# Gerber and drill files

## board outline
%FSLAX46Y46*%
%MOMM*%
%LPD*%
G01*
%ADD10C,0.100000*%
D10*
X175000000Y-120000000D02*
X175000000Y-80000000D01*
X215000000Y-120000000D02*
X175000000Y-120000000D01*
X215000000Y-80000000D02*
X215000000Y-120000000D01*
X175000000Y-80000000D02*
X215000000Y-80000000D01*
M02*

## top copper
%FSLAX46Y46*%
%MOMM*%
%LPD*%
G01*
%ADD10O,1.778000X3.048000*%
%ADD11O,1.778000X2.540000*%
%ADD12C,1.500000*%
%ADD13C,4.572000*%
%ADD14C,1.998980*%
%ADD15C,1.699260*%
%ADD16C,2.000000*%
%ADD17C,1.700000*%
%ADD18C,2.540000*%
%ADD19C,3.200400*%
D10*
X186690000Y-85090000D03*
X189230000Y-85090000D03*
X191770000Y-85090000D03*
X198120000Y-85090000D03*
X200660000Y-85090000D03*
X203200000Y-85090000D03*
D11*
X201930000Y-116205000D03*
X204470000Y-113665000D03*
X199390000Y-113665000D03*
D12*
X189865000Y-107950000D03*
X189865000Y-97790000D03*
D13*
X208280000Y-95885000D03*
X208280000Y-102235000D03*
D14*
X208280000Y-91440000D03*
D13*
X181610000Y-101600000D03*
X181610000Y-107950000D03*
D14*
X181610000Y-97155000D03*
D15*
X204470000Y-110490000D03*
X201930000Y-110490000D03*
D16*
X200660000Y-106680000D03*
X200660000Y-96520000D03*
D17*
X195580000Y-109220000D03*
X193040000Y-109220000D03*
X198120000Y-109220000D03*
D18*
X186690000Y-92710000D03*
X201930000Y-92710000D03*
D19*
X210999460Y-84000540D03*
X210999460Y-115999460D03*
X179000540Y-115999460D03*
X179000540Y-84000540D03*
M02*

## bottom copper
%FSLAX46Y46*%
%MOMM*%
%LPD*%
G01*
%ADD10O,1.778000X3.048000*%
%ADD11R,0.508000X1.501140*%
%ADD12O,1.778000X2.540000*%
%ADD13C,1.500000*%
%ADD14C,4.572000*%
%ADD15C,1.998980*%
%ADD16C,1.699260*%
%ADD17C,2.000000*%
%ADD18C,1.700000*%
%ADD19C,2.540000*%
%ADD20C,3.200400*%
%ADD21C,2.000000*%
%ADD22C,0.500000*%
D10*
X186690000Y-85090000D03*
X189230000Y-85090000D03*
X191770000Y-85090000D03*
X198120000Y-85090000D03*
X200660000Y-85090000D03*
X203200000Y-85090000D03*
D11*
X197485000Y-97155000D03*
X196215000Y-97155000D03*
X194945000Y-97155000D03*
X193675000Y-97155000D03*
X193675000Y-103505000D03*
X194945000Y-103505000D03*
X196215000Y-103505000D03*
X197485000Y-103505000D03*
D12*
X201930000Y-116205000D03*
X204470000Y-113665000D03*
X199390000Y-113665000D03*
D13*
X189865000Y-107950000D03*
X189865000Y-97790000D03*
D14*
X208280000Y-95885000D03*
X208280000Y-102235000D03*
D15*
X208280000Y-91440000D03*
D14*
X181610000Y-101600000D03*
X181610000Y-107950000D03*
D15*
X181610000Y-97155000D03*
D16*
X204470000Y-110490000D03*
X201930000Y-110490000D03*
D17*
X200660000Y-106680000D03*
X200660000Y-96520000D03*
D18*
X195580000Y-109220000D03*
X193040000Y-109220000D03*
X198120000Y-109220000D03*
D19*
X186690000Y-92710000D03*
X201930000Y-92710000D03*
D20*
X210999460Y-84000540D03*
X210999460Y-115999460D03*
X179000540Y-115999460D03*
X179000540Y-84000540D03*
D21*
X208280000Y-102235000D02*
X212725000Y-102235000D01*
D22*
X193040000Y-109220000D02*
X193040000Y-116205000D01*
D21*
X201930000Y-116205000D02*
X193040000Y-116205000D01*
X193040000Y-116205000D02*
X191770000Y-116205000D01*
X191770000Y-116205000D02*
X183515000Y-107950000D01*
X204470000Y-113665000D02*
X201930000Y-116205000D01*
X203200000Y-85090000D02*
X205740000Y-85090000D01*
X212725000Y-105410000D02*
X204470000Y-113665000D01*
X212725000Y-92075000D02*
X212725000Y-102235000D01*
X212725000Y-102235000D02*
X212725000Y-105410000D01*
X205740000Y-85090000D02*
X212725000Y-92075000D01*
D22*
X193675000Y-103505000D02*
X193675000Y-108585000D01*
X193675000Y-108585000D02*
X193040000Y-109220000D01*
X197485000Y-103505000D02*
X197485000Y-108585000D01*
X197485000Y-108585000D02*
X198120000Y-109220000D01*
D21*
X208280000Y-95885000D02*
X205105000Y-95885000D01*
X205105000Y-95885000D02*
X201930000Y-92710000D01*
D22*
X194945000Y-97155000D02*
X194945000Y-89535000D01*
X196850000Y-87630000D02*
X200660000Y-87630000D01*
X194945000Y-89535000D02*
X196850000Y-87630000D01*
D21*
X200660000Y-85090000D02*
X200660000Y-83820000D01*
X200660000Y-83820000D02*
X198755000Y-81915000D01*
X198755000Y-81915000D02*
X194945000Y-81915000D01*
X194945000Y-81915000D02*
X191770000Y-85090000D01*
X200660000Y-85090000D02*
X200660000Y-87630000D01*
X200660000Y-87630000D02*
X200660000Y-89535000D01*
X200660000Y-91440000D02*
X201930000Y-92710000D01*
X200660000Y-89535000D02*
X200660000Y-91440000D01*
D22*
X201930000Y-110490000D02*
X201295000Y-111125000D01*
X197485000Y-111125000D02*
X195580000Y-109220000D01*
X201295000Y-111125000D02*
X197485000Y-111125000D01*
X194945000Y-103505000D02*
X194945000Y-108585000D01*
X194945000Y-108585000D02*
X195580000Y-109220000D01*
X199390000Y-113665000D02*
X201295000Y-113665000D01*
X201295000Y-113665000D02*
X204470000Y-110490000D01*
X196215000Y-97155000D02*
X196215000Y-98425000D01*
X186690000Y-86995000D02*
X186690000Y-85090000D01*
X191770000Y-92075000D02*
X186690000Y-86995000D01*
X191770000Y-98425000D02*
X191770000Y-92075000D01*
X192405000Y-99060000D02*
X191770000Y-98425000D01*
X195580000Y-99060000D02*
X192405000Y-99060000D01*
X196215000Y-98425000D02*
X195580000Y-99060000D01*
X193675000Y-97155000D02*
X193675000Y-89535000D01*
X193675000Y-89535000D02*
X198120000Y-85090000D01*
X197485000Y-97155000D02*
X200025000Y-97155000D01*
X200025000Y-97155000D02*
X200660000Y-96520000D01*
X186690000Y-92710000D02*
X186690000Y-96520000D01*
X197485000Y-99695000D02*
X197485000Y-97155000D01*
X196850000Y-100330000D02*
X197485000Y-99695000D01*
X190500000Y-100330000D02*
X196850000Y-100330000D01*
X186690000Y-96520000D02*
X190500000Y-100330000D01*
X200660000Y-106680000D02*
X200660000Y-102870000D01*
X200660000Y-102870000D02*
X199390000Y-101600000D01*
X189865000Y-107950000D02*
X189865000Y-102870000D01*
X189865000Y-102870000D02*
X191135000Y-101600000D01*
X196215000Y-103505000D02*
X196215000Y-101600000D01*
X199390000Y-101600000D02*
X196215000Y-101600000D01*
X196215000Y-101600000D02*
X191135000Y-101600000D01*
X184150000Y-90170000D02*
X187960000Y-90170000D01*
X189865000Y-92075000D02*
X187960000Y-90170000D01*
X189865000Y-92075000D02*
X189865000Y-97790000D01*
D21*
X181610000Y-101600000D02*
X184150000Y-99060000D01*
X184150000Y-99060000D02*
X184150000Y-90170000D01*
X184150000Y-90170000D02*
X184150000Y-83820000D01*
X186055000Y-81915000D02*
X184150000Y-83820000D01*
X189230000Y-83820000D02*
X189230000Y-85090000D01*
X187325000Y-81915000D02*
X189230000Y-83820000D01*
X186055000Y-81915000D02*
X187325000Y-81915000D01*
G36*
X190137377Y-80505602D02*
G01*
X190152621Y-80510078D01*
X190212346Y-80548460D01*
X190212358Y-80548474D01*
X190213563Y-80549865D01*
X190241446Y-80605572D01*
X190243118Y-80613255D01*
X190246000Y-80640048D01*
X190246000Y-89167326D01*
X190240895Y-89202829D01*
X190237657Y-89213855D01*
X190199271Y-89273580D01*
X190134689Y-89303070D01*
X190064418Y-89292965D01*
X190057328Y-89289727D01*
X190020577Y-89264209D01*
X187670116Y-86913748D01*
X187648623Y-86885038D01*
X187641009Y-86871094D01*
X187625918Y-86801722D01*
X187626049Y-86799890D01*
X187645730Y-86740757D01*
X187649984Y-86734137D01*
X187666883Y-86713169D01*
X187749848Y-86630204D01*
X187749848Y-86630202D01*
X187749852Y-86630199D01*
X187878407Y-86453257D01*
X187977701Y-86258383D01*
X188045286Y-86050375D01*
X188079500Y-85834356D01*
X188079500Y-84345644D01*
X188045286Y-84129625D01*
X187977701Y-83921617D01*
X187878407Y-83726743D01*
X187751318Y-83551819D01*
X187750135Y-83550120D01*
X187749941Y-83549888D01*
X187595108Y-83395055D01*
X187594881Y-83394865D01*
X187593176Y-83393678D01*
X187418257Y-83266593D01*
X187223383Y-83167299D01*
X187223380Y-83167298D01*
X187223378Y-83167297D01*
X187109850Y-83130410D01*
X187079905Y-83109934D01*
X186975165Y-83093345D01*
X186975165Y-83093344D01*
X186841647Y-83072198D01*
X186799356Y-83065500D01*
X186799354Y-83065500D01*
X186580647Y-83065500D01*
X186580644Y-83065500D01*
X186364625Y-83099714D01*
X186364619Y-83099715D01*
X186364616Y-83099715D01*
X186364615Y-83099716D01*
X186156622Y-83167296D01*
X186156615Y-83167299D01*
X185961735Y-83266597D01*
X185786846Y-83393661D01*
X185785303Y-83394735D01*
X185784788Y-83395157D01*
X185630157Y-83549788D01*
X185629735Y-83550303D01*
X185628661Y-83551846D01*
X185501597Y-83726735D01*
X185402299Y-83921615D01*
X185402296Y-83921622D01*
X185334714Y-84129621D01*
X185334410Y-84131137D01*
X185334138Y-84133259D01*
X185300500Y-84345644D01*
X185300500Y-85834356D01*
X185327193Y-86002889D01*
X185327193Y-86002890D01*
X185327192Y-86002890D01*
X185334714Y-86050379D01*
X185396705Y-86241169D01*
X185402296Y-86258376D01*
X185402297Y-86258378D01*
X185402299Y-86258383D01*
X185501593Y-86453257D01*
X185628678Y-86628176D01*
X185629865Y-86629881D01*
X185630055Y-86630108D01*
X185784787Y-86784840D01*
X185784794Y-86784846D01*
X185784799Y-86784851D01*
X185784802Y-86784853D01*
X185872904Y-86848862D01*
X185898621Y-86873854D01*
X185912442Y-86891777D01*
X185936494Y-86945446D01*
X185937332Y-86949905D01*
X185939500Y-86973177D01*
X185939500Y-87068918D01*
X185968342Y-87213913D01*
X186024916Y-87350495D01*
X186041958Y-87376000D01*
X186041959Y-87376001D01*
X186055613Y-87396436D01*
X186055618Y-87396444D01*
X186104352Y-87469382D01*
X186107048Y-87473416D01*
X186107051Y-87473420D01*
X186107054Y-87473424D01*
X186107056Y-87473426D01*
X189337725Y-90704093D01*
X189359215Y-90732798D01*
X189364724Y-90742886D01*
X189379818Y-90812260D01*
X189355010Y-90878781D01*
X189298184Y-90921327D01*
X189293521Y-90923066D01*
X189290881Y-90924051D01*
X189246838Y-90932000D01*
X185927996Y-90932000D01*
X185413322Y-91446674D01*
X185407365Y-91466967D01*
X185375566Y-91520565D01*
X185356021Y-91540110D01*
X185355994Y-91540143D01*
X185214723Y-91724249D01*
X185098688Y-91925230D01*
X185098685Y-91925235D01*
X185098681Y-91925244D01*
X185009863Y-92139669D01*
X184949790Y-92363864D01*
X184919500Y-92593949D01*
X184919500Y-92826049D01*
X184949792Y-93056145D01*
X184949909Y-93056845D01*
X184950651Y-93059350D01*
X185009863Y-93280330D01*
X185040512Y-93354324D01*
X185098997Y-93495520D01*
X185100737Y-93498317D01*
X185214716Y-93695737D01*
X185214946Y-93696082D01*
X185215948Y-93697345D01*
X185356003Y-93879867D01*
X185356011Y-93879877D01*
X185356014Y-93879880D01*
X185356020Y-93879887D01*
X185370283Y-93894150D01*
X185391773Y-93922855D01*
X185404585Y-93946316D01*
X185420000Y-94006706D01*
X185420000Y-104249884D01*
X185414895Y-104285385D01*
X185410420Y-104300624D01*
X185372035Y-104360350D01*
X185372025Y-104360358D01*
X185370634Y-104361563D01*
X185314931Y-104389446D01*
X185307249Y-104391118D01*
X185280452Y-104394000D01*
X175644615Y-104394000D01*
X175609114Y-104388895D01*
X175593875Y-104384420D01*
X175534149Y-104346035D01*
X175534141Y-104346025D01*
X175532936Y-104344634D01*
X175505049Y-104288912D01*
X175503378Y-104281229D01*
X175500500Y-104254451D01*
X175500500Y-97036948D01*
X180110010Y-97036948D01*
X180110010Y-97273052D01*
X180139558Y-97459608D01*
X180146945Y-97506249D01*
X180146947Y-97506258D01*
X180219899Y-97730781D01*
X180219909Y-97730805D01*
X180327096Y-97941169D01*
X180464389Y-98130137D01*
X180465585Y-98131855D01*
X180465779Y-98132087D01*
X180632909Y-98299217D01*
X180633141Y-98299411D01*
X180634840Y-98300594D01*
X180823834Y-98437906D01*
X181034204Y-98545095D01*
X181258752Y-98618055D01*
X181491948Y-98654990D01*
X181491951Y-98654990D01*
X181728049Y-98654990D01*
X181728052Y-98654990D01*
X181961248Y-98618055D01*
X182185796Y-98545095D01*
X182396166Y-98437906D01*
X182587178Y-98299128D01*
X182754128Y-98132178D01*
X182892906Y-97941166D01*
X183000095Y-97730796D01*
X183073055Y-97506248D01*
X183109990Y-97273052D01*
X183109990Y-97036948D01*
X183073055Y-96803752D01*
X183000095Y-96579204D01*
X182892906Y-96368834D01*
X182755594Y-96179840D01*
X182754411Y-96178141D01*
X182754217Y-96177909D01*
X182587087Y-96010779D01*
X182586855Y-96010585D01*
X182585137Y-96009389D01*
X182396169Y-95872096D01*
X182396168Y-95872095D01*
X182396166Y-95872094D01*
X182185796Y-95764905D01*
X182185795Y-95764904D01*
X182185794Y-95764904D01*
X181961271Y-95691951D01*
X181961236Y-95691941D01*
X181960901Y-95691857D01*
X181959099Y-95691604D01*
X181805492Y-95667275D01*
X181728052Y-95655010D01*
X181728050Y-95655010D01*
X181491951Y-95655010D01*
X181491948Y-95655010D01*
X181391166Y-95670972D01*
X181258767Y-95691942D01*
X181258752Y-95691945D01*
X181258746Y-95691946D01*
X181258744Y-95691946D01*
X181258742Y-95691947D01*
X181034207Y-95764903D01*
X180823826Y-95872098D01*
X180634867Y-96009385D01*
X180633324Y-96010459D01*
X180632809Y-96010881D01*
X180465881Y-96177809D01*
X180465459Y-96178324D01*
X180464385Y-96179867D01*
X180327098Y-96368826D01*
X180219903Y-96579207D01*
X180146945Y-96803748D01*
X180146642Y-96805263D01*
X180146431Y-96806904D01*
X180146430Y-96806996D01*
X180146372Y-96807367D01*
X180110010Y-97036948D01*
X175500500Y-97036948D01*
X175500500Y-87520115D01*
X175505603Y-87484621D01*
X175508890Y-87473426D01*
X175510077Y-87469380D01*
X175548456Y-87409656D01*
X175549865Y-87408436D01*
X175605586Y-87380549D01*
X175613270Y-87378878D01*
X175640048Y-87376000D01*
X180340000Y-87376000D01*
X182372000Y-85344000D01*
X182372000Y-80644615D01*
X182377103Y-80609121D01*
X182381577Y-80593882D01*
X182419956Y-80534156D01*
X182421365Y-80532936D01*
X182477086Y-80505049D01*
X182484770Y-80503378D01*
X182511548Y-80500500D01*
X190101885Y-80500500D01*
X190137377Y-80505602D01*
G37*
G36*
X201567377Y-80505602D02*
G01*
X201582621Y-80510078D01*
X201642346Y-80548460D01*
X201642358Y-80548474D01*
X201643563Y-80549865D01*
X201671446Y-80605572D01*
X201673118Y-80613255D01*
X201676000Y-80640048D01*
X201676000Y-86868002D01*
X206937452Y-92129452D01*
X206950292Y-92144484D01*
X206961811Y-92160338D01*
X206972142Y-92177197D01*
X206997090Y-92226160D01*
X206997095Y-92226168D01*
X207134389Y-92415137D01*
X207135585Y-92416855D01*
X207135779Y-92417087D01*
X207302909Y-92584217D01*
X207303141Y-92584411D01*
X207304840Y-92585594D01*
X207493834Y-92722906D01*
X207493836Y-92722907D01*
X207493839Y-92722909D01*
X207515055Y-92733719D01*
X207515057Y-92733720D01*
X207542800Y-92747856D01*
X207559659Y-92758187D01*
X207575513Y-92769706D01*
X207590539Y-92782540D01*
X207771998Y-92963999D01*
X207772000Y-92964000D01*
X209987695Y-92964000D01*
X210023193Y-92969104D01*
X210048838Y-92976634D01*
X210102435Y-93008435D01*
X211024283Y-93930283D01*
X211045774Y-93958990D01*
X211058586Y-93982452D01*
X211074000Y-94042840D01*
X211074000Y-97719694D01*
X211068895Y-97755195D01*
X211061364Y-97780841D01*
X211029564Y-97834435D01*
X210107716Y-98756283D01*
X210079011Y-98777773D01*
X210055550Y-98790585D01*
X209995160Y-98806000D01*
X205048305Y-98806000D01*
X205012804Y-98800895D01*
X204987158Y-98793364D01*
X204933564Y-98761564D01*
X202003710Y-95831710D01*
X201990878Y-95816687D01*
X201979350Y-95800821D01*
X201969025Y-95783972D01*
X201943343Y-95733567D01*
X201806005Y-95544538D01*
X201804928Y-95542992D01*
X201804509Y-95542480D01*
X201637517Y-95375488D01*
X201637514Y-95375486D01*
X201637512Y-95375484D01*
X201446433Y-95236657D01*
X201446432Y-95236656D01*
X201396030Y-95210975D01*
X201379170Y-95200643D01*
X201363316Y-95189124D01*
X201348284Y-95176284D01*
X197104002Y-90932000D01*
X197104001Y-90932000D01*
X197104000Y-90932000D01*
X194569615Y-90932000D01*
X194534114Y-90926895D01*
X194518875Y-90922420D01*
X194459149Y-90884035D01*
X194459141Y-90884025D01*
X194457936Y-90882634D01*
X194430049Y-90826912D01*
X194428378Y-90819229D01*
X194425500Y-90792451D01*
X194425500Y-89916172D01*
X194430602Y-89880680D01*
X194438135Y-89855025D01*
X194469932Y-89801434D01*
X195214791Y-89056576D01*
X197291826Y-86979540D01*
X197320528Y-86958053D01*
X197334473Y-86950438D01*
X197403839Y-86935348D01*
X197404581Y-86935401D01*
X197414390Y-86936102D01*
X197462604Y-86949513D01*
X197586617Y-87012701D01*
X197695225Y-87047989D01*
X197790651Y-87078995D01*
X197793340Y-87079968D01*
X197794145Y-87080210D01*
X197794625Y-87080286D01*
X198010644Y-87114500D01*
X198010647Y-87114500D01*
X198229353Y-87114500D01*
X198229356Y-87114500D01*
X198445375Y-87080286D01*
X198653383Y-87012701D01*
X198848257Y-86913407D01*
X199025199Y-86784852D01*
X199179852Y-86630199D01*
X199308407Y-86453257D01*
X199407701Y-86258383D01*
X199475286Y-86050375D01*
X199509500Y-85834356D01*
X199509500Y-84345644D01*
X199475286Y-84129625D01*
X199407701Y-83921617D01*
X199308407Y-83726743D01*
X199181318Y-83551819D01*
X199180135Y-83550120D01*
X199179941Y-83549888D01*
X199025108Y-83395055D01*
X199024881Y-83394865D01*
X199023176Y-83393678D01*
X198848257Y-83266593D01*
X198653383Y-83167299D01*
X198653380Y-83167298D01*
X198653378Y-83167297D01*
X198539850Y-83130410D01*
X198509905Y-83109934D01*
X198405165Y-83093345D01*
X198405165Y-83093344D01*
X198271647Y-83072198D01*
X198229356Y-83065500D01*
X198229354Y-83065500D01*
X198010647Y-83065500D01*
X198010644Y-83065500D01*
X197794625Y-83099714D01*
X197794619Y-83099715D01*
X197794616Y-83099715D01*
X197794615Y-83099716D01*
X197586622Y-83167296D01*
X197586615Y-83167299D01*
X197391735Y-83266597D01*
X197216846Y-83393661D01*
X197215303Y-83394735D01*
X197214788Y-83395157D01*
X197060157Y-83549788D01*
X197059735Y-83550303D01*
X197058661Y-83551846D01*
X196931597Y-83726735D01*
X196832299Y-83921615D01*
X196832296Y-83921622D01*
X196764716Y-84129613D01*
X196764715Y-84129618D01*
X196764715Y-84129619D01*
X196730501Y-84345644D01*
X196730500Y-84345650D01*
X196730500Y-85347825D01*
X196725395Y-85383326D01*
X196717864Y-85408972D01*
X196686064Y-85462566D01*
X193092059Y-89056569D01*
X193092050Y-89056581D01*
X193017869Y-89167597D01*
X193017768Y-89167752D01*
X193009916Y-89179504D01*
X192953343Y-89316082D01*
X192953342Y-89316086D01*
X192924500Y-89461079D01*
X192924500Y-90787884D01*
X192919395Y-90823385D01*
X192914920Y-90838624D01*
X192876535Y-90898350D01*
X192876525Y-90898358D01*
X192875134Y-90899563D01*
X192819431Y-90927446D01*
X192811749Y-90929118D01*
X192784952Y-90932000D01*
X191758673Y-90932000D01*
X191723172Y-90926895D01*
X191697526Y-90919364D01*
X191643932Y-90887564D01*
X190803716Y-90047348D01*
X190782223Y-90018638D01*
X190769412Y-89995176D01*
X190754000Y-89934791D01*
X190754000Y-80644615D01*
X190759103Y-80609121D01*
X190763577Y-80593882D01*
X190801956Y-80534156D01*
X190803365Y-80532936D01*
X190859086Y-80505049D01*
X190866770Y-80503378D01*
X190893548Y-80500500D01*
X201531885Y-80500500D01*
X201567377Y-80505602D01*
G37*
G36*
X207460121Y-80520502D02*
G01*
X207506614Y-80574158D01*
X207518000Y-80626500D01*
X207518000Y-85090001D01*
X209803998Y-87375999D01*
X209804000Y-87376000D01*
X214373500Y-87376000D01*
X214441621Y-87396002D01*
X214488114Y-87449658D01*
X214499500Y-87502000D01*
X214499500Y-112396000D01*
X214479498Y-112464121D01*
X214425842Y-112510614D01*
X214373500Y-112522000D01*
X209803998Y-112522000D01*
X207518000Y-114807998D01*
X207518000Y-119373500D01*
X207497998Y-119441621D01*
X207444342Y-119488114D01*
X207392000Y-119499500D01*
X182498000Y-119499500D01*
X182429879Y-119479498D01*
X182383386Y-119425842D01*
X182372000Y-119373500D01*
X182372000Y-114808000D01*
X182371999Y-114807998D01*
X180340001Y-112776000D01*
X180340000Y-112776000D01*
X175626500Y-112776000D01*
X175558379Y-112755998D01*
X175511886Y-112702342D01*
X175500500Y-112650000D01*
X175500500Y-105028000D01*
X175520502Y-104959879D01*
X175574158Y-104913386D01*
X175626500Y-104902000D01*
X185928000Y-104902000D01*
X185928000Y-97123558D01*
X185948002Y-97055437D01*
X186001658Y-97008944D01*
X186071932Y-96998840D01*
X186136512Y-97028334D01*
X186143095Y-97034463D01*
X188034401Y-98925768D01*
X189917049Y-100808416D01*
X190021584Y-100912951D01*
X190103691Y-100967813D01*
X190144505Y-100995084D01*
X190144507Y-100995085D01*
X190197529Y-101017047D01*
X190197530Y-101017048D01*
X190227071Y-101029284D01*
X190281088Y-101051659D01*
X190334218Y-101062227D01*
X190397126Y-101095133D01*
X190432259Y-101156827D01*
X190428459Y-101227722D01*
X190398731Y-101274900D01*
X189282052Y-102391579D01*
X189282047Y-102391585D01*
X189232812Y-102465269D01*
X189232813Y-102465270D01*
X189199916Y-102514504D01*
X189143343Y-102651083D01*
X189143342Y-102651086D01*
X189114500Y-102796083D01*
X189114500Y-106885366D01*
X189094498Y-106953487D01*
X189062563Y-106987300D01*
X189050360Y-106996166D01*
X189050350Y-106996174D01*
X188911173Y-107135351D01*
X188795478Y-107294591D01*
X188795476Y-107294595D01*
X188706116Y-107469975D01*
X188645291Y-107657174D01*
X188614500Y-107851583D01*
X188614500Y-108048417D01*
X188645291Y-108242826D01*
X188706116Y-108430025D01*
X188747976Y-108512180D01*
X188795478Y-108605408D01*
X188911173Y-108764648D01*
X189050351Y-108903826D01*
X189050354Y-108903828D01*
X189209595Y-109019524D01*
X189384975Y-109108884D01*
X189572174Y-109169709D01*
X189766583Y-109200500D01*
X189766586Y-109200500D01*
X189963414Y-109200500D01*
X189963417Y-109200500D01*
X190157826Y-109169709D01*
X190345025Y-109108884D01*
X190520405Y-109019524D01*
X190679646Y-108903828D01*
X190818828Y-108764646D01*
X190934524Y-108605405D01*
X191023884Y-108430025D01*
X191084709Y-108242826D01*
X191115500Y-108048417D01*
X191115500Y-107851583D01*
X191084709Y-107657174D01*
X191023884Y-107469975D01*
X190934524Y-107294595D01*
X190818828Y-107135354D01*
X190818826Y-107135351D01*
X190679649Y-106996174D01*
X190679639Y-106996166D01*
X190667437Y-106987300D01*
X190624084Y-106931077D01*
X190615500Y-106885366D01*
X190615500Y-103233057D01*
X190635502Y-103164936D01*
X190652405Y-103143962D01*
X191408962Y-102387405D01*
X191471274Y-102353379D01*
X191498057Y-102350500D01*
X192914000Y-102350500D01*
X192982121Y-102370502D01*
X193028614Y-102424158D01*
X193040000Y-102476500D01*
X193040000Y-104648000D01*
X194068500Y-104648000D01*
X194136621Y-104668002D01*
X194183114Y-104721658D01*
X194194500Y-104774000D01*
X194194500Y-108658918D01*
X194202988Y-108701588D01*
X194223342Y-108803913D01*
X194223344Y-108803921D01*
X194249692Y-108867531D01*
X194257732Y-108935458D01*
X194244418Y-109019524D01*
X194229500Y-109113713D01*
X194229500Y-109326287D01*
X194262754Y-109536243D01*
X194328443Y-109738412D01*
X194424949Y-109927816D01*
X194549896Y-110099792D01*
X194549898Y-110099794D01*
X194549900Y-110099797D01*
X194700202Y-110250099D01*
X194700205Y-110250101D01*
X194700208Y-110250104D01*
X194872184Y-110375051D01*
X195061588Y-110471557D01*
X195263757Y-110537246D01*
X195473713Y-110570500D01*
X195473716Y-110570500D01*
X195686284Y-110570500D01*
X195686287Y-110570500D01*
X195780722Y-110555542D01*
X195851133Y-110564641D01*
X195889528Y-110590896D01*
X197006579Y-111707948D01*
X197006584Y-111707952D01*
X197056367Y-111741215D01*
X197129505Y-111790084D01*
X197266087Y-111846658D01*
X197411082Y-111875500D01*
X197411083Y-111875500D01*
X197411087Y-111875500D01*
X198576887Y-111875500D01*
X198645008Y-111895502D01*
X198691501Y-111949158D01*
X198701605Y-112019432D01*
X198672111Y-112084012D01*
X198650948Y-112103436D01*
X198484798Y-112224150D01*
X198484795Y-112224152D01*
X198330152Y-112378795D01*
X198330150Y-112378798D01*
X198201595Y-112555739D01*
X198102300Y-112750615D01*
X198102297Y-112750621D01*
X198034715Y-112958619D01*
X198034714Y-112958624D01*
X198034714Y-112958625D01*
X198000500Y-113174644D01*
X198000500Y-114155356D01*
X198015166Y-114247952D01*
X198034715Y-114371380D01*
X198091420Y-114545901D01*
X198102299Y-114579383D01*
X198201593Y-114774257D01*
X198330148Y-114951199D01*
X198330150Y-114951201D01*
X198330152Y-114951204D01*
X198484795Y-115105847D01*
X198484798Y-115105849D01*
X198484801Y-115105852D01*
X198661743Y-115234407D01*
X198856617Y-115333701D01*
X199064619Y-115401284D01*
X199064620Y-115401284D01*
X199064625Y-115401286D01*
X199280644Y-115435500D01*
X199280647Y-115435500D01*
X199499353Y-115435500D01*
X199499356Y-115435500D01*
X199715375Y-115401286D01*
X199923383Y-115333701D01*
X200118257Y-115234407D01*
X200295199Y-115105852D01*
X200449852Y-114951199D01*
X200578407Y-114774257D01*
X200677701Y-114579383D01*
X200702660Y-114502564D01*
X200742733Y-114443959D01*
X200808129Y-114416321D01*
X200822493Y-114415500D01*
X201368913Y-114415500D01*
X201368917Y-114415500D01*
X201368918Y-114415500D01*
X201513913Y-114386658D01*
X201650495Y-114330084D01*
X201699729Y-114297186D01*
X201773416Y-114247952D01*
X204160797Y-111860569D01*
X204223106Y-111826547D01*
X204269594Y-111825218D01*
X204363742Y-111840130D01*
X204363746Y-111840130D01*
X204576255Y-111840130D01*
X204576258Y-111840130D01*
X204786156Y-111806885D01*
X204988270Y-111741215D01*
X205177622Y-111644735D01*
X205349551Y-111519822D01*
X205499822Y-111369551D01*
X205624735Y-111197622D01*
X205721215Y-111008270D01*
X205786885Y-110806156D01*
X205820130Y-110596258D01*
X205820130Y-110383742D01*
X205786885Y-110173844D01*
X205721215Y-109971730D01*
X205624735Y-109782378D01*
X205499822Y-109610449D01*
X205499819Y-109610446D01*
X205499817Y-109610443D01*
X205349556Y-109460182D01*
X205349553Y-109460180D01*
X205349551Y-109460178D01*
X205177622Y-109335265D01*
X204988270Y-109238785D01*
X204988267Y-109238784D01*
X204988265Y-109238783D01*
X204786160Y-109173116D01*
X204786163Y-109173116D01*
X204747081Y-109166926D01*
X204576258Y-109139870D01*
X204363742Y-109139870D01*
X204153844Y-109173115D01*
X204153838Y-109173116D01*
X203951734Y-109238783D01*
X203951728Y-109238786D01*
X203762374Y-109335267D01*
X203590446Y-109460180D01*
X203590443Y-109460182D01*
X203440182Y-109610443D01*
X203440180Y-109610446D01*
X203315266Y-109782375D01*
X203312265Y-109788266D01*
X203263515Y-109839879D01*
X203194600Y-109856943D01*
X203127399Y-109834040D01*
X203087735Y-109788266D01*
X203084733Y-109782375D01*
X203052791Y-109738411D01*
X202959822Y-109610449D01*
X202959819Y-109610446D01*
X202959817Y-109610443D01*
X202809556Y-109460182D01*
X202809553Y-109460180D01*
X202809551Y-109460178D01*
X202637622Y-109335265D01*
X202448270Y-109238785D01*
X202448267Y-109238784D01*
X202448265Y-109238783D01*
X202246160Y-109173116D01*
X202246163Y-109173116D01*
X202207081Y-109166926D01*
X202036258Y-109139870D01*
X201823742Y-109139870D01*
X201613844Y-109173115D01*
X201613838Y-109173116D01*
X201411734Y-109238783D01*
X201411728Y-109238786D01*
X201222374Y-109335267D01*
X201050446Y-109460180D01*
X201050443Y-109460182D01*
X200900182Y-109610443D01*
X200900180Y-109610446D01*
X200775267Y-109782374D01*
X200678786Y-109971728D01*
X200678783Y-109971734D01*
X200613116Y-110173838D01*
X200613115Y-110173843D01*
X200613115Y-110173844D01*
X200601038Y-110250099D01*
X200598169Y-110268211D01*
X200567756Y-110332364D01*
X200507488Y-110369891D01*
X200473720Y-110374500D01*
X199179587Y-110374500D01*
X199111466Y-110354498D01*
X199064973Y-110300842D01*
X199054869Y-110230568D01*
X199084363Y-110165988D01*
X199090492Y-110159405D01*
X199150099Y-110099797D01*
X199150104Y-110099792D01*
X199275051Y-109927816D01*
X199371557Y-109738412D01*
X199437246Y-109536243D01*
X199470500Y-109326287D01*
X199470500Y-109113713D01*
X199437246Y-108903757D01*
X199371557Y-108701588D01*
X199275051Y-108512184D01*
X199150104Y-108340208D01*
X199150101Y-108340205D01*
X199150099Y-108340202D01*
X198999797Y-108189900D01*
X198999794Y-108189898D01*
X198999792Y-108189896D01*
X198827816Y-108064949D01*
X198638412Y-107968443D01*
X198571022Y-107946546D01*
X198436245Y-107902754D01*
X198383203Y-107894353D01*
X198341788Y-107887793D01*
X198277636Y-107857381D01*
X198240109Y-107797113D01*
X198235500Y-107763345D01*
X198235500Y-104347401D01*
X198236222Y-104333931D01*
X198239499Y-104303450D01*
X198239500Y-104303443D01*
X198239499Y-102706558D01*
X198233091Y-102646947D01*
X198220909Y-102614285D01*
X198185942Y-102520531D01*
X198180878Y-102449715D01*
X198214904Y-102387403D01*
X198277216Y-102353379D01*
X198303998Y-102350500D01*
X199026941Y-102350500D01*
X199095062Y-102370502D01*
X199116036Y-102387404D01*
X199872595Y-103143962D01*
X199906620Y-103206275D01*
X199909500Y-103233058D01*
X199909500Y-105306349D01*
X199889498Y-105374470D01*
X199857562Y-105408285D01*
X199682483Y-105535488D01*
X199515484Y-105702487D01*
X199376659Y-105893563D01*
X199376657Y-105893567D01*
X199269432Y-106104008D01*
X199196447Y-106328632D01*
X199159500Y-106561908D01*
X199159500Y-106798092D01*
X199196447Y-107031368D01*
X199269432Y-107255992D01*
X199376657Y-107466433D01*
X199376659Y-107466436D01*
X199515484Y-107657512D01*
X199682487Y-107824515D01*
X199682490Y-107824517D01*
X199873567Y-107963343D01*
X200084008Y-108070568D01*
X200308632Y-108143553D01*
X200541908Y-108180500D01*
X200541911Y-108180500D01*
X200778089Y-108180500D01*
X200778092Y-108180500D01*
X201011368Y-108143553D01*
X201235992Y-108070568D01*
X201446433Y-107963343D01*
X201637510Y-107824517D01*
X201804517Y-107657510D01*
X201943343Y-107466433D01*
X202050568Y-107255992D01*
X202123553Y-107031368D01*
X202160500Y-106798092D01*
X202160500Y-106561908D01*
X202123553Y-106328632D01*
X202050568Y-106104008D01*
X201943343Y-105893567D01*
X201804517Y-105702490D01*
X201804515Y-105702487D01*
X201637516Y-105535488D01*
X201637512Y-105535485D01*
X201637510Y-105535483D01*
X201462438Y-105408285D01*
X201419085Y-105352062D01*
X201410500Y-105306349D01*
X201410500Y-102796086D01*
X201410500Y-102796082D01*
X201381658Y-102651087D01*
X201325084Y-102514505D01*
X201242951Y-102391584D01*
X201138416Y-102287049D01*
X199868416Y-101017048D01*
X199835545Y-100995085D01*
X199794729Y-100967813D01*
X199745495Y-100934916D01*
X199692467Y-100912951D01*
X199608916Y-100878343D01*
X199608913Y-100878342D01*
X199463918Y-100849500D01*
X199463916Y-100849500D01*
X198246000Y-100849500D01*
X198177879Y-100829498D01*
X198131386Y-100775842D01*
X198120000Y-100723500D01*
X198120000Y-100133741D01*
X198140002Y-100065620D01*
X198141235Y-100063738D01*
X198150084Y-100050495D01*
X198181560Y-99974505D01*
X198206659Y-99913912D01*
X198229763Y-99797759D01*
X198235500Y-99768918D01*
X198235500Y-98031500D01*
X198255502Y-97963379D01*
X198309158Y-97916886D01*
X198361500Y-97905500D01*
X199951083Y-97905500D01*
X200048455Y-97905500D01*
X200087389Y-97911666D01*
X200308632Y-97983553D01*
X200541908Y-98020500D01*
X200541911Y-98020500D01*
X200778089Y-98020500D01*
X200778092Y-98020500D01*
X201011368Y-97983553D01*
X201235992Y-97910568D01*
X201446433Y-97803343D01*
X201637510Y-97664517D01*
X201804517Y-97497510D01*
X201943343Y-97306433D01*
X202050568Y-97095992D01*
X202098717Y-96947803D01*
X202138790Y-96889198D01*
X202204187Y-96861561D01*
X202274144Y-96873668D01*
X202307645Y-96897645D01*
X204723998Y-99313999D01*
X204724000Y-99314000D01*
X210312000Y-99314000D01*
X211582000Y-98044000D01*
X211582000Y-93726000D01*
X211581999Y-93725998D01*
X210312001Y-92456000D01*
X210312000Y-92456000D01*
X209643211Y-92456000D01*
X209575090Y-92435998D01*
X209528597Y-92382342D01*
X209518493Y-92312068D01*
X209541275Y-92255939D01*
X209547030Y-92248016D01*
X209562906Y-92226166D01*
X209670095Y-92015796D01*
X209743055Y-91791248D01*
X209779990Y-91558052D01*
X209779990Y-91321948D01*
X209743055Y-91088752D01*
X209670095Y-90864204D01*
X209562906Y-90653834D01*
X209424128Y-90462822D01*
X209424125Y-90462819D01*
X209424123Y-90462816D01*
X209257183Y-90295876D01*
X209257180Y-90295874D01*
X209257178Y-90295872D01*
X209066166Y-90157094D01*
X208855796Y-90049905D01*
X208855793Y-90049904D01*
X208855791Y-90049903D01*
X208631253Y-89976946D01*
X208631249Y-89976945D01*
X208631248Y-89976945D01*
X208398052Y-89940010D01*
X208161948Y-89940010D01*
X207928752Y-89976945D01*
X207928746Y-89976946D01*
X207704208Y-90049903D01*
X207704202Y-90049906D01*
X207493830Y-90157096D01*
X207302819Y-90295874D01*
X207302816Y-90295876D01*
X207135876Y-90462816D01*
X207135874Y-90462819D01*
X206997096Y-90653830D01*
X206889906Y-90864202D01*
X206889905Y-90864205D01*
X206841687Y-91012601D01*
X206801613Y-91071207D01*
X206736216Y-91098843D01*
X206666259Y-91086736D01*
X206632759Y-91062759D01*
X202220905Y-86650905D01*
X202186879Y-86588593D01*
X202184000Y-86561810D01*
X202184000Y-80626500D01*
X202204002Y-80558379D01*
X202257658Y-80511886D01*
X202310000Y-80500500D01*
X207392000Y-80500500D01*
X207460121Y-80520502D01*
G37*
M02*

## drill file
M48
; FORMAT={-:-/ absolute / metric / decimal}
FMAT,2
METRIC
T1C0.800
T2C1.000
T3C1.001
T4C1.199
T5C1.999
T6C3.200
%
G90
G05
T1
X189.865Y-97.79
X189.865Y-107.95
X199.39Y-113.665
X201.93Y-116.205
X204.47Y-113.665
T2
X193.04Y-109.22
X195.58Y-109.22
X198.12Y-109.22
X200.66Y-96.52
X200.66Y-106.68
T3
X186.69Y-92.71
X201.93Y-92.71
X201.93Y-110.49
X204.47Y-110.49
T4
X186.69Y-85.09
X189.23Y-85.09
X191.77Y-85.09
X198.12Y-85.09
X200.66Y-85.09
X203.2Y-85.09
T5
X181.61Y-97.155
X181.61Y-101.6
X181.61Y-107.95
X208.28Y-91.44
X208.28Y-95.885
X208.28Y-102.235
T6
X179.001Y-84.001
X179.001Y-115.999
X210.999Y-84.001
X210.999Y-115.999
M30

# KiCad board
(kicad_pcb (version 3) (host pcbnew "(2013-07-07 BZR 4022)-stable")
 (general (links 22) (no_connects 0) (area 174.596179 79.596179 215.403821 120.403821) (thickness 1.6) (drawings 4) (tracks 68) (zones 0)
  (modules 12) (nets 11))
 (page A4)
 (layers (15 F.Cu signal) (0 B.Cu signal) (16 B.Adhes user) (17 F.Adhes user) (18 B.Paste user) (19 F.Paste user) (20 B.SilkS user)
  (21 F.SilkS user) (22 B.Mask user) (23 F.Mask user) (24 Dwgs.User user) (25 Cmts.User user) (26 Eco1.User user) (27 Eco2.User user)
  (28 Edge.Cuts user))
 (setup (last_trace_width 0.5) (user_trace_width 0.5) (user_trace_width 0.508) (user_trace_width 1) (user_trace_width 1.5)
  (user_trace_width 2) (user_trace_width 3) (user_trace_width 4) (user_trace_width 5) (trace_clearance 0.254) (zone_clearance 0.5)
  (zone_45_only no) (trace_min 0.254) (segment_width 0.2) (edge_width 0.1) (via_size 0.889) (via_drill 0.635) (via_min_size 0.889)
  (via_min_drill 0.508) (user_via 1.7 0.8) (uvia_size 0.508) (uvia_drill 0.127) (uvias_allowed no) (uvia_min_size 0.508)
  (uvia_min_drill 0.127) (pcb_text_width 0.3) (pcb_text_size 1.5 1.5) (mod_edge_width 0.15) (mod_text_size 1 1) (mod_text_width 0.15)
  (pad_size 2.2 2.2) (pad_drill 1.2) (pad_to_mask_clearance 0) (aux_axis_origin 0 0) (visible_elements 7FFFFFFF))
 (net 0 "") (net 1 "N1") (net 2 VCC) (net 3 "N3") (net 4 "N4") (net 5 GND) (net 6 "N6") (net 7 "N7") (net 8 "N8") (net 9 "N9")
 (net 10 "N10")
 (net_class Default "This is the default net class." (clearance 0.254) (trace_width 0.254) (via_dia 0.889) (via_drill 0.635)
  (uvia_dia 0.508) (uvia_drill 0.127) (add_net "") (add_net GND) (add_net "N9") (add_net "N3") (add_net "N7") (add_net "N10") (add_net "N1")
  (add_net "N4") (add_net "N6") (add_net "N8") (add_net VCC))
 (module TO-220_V (layer F.Cu) (at 189.23 85.09 90)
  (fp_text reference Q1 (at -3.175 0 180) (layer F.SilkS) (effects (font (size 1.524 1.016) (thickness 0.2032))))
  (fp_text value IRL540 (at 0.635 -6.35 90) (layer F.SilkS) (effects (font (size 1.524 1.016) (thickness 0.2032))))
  (pad 1 thru_hole oval (at 0 -2.54 90) (size 3.048 1.778) (drill 1.19888) (layers *.Cu *.Mask F.SilkS) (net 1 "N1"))
  (pad 2 thru_hole oval (at 0 0 90) (size 3.048 1.778) (drill 1.19888) (layers *.Cu *.Mask F.SilkS) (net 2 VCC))
  (pad 3 thru_hole oval (at 0 2.54 90) (size 3.048 1.778) (drill 1.19888) (layers *.Cu *.Mask F.SilkS) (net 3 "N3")))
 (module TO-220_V (layer F.Cu) (at 200.66 85.09 90)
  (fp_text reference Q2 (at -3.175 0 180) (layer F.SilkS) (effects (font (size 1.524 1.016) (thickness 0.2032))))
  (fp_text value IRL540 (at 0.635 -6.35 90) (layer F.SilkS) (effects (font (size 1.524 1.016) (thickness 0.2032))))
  (pad 1 thru_hole oval (at 0 -2.54 90) (size 3.048 1.778) (drill 1.19888) (layers *.Cu *.Mask F.SilkS) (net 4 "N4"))
  (pad 2 thru_hole oval (at 0 0 90) (size 3.048 1.778) (drill 1.19888) (layers *.Cu *.Mask F.SilkS) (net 3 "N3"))
  (pad 3 thru_hole oval (at 0 2.54 90) (size 3.048 1.778) (drill 1.19888) (layers *.Cu *.Mask F.SilkS) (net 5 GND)))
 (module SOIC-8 (layer B.Cu) (at 195.58 100.33 180)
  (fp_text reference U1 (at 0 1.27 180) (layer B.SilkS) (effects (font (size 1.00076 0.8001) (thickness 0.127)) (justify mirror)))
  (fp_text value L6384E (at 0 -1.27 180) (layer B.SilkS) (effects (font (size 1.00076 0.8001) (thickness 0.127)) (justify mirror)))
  (pad 8 smd rect (at -1.905 3.175 180) (size 0.508 1.50114) (layers B.Cu B.Paste B.Mask) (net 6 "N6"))
  (pad 7 smd rect (at -0.635 3.175 180) (size 0.508 1.50114) (layers B.Cu B.Paste B.Mask) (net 1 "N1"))
  (pad 6 smd rect (at 0.635 3.175 180) (size 0.508 1.50114) (layers B.Cu B.Paste B.Mask) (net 3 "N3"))
  (pad 5 smd rect (at 1.905 3.175 180) (size 0.508 1.50114) (layers B.Cu B.Paste B.Mask) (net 4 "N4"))
  (pad 4 smd rect (at 1.905 -3.175 180) (size 0.508 1.50114) (layers B.Cu B.Paste B.Mask) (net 5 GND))
  (pad 3 smd rect (at 0.635 -3.175 180) (size 0.508 1.50114) (layers B.Cu B.Paste B.Mask) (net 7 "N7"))
  (pad 2 smd rect (at -0.635 -3.175 180) (size 0.508 1.50114) (layers B.Cu B.Paste B.Mask) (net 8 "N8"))
  (pad 1 smd rect (at -1.905 -3.175 180) (size 0.508 1.50114) (layers B.Cu B.Paste B.Mask) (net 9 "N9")))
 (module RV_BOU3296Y (layer F.Cu) (at 201.93 114.935 180)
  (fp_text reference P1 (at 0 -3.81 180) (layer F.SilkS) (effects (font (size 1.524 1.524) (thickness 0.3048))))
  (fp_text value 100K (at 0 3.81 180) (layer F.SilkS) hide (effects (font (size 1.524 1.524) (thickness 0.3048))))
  (pad 2 thru_hole oval (at 0 -1.27 180) (size 1.778 2.54) (drill 0.8001) (layers *.Cu *.Mask F.SilkS) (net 5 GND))
  (pad 1 thru_hole oval (at -2.54 1.27 180) (size 1.778 2.54) (drill 0.8001) (layers *.Cu *.Mask F.SilkS) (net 5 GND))
  (pad 3 thru_hole oval (at 2.54 1.27 180) (size 1.778 2.54) (drill 0.8001) (layers *.Cu *.Mask F.SilkS) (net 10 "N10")))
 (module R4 (layer F.Cu) (at 189.865 102.87 90) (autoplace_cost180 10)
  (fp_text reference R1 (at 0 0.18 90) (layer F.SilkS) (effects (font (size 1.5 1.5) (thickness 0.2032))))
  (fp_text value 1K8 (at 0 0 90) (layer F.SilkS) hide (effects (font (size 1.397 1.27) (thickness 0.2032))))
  (pad 1 thru_hole circle (at -5.08 0 90) (size 1.5 1.5) (drill 0.8001) (layers *.Cu *.Mask F.SilkS) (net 8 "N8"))
  (pad 2 thru_hole circle (at 5.08 0 90) (size 1.5 1.5) (drill 0.8001) (layers *.Cu *.Mask F.SilkS) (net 2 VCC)))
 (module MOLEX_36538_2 (layer F.Cu) (at 208.28 99.06 270)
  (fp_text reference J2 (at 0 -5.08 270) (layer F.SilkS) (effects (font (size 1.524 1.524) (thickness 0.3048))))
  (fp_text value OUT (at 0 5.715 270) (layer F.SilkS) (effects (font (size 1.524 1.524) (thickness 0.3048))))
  (pad 1 thru_hole circle (at -3.175 0 270) (size 4.572 4.572) (drill 1.99898) (layers *.Cu *.Mask F.SilkS) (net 3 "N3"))
  (pad 2 thru_hole circle (at 3.175 0 270) (size 4.572 4.572) (drill 1.99898) (layers *.Cu *.Mask F.SilkS) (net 5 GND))
  (pad "" thru_hole circle (at -7.62 0 270) (size 1.99898 1.99898) (drill 1.99898) (layers *.Cu *.Mask F.SilkS)))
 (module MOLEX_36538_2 (layer F.Cu) (at 181.61 104.775 270)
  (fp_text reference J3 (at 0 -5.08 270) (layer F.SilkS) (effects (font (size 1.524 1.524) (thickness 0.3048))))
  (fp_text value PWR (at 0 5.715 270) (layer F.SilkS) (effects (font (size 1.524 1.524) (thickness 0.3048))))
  (pad 1 thru_hole circle (at -3.175 0 270) (size 4.572 4.572) (drill 1.99898) (layers *.Cu *.Mask F.SilkS) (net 2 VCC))
  (pad 2 thru_hole circle (at 3.175 0 270) (size 4.572 4.572) (drill 1.99898) (layers *.Cu *.Mask F.SilkS) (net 5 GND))
  (pad "" thru_hole circle (at -7.62 0 270) (size 1.99898 1.99898) (drill 1.99898) (layers *.Cu *.Mask F.SilkS)))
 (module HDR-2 (layer F.Cu) (at 203.2 110.49 180)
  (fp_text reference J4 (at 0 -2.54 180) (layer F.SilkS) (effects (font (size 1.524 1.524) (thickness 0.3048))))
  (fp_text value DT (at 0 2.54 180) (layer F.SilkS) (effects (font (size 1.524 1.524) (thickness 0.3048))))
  (pad 1 thru_hole circle (at -1.27 0 180) (size 1.69926 1.69926) (drill 1.00076) (layers *.Cu *.Mask F.SilkS) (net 10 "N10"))
  (pad 2 thru_hole circle (at 1.27 0 180) (size 1.69926 1.69926) (drill 1.00076) (layers *.Cu *.Mask F.SilkS) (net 7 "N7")))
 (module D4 (layer F.Cu) (at 200.66 101.6 90)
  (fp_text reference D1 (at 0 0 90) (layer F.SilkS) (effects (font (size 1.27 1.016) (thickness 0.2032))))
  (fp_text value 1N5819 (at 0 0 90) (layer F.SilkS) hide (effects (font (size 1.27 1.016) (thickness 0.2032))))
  (pad 1 thru_hole circle (at -5.08 0 90) (size 2 2) (drill 1) (layers *.Cu *.Mask F.SilkS) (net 8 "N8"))
  (pad 2 thru_hole circle (at 5.08 0 90) (size 2 2) (drill 1) (layers *.Cu *.Mask F.SilkS) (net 6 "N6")))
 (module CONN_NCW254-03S (layer F.Cu) (at 195.58 109.22 180)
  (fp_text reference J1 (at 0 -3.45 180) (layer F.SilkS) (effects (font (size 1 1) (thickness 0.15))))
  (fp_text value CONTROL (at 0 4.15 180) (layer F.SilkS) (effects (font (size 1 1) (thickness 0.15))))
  (pad 2 thru_hole circle (at 0 0 180) (size 1.7 1.7) (drill 1) (layers *.Cu *.Mask F.SilkS) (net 7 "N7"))
  (pad 3 thru_hole circle (at 2.54 0 180) (size 1.7 1.7) (drill 1) (layers *.Cu *.Mask F.SilkS) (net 5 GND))
  (pad 1 thru_hole circle (at -2.54 0 180) (size 1.7 1.7) (drill 1) (layers *.Cu *.Mask F.SilkS) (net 9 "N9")))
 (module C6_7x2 (layer F.Cu) (at 194.31 92.71)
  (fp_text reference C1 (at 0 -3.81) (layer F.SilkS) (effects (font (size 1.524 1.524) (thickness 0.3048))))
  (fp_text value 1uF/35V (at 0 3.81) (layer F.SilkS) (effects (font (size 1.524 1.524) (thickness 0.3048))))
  (pad 1 thru_hole circle (at -7.62 0) (size 2.54 2.54) (drill 1.00076) (layers *.Cu *.Mask F.SilkS) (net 6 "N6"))
  (pad 2 thru_hole circle (at 7.62 0) (size 2.54 2.54) (drill 1.00076) (layers *.Cu *.Mask F.SilkS) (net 3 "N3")))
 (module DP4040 (layer F.Cu) (at 195 100)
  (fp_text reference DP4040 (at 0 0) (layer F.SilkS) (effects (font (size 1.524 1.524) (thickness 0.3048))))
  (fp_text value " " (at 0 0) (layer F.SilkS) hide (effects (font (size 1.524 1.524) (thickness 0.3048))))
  (pad "" thru_hole circle (at 15.99946 -15.99946) (size 3.2004 3.2004) (drill 3.2004) (layers *.Cu *.Mask F.SilkS) (clearance 1.39954))
  (pad "" thru_hole circle (at 15.99946 15.99946) (size 3.2004 3.2004) (drill 3.2004) (layers *.Cu *.Mask F.SilkS) (clearance 1.39954))
  (pad "" thru_hole circle (at -15.99946 15.99946) (size 3.2004 3.2004) (drill 3.2004) (layers *.Cu *.Mask F.SilkS) (clearance 1.39954))
  (pad "" thru_hole circle (at -15.99946 -15.99946) (size 3.2004 3.2004) (drill 3.2004) (layers *.Cu *.Mask F.SilkS) (clearance 1.39954)))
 (gr_line (start 175 120) (end 175 80) (angle 90) (layer Edge.Cuts) (width 0.1))
 (gr_line (start 215 120) (end 175 120) (angle 90) (layer Edge.Cuts) (width 0.1))
 (gr_line (start 215 80) (end 215 120) (angle 90) (layer Edge.Cuts) (width 0.1))
 (gr_line (start 175 80) (end 215 80) (angle 90) (layer Edge.Cuts) (width 0.1))
 (segment (start 208.28 102.235) (end 212.725 102.235) (width 2) (layer B.Cu) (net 5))
 (segment (start 193.04 109.22) (end 193.04 116.205) (width 0.5) (layer B.Cu) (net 5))
 (segment (start 201.93 116.205) (end 193.04 116.205) (width 2) (layer B.Cu) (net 5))
 (segment (start 193.04 116.205) (end 191.77 116.205) (width 2) (layer B.Cu) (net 5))
 (segment (start 191.77 116.205) (end 183.515 107.95) (width 2) (layer B.Cu) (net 5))
 (segment (start 204.47 113.665) (end 201.93 116.205) (width 2) (layer B.Cu) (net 5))
 (segment (start 203.2 85.09) (end 205.74 85.09) (width 2) (layer B.Cu) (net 5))
 (segment (start 212.725 105.41) (end 204.47 113.665) (width 2) (layer B.Cu) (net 5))
 (segment (start 212.725 92.075) (end 212.725 102.235) (width 2) (layer B.Cu) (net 5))
 (segment (start 212.725 102.235) (end 212.725 105.41) (width 2) (layer B.Cu) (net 5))
 (segment (start 205.74 85.09) (end 212.725 92.075) (width 2) (layer B.Cu) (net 5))
 (segment (start 193.675 103.505) (end 193.675 108.585) (width 0.5) (layer B.Cu) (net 5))
 (segment (start 193.675 108.585) (end 193.04 109.22) (width 0.5) (layer B.Cu) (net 5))
 (segment (start 197.485 103.505) (end 197.485 108.585) (width 0.5) (layer B.Cu) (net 9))
 (segment (start 197.485 108.585) (end 198.12 109.22) (width 0.5) (layer B.Cu) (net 9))
 (segment (start 208.28 95.885) (end 205.105 95.885) (width 2) (layer B.Cu) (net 3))
 (segment (start 205.105 95.885) (end 201.93 92.71) (width 2) (layer B.Cu) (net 3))
 (segment (start 194.945 97.155) (end 194.945 89.535) (width 0.5) (layer B.Cu) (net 3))
 (segment (start 196.85 87.63) (end 200.66 87.63) (width 0.5) (layer B.Cu) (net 3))
 (segment (start 194.945 89.535) (end 196.85 87.63) (width 0.5) (layer B.Cu) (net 3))
 (segment (start 200.66 85.09) (end 200.66 83.82) (width 2) (layer B.Cu) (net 3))
 (segment (start 200.66 83.82) (end 198.755 81.915) (width 2) (layer B.Cu) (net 3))
 (segment (start 198.755 81.915) (end 194.945 81.915) (width 2) (layer B.Cu) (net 3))
 (segment (start 194.945 81.915) (end 191.77 85.09) (width 2) (layer B.Cu) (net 3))
 (segment (start 200.66 85.09) (end 200.66 87.63) (width 2) (layer B.Cu) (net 3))
 (segment (start 200.66 87.63) (end 200.66 89.535) (width 2) (layer B.Cu) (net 3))
 (segment (start 200.66 91.44) (end 201.93 92.71) (width 2) (layer B.Cu) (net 3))
 (segment (start 200.66 89.535) (end 200.66 91.44) (width 2) (layer B.Cu) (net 3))
 (segment (start 201.93 110.49) (end 201.295 111.125) (width 0.5) (layer B.Cu) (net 7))
 (segment (start 197.485 111.125) (end 195.58 109.22) (width 0.5) (layer B.Cu) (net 7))
 (segment (start 201.295 111.125) (end 197.485 111.125) (width 0.5) (layer B.Cu) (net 7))
 (segment (start 194.945 103.505) (end 194.945 108.585) (width 0.5) (layer B.Cu) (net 7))
 (segment (start 194.945 108.585) (end 195.58 109.22) (width 0.5) (layer B.Cu) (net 7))
 (segment (start 199.39 113.665) (end 201.295 113.665) (width 0.5) (layer B.Cu) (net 10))
 (segment (start 201.295 113.665) (end 204.47 110.49) (width 0.5) (layer B.Cu) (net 10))
 (segment (start 196.215 97.155) (end 196.215 98.425) (width 0.5) (layer B.Cu) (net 1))
 (segment (start 186.69 86.995) (end 186.69 85.09) (width 0.5) (layer B.Cu) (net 1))
 (segment (start 191.77 92.075) (end 186.69 86.995) (width 0.5) (layer B.Cu) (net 1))
 (segment (start 191.77 98.425) (end 191.77 92.075) (width 0.5) (layer B.Cu) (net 1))
 (segment (start 192.405 99.06) (end 191.77 98.425) (width 0.5) (layer B.Cu) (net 1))
 (segment (start 195.58 99.06) (end 192.405 99.06) (width 0.5) (layer B.Cu) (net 1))
 (segment (start 196.215 98.425) (end 195.58 99.06) (width 0.5) (layer B.Cu) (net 1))
 (segment (start 193.675 97.155) (end 193.675 89.535) (width 0.5) (layer B.Cu) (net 4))
 (segment (start 193.675 89.535) (end 198.12 85.09) (width 0.5) (layer B.Cu) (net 4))
 (segment (start 197.485 97.155) (end 200.025 97.155) (width 0.5) (layer B.Cu) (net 6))
 (segment (start 200.025 97.155) (end 200.66 96.52) (width 0.5) (layer B.Cu) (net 6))
 (segment (start 186.69 92.71) (end 186.69 96.52) (width 0.5) (layer B.Cu) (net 6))
 (segment (start 197.485 99.695) (end 197.485 97.155) (width 0.5) (layer B.Cu) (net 6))
 (segment (start 196.85 100.33) (end 197.485 99.695) (width 0.5) (layer B.Cu) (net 6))
 (segment (start 190.5 100.33) (end 196.85 100.33) (width 0.5) (layer B.Cu) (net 6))
 (segment (start 186.69 96.52) (end 190.5 100.33) (width 0.5) (layer B.Cu) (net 6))
 (segment (start 200.66 106.68) (end 200.66 102.87) (width 0.5) (layer B.Cu) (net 8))
 (segment (start 200.66 102.87) (end 199.39 101.6) (width 0.5) (layer B.Cu) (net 8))
 (segment (start 189.865 107.95) (end 189.865 102.87) (width 0.5) (layer B.Cu) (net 8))
 (segment (start 189.865 102.87) (end 191.135 101.6) (width 0.5) (layer B.Cu) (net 8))
 (segment (start 196.215 103.505) (end 196.215 101.6) (width 0.5) (layer B.Cu) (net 8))
 (segment (start 199.39 101.6) (end 196.215 101.6) (width 0.5) (layer B.Cu) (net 8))
 (segment (start 196.215 101.6) (end 191.135 101.6) (width 0.5) (layer B.Cu) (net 8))
 (segment (start 184.15 90.17) (end 187.96 90.17) (width 0.5) (layer B.Cu) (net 2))
 (segment (start 189.865 92.075) (end 187.96 90.17) (width 0.5) (layer B.Cu) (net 2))
 (segment (start 189.865 92.075) (end 189.865 97.79) (width 0.5) (layer B.Cu) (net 2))
 (segment (start 181.61 101.6) (end 184.15 99.06) (width 2) (layer B.Cu) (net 2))
 (segment (start 184.15 99.06) (end 184.15 90.17) (width 2) (layer B.Cu) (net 2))
 (segment (start 184.15 90.17) (end 184.15 83.82) (width 2) (layer B.Cu) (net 2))
 (segment (start 186.055 81.915) (end 184.15 83.82) (width 2) (layer B.Cu) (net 2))
 (segment (start 189.23 83.82) (end 189.23 85.09) (width 2) (layer B.Cu) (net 2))
 (segment (start 187.325 81.915) (end 189.23 83.82) (width 2) (layer B.Cu) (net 2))
 (segment (start 186.055 81.915) (end 187.325 81.915) (width 2) (layer B.Cu) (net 2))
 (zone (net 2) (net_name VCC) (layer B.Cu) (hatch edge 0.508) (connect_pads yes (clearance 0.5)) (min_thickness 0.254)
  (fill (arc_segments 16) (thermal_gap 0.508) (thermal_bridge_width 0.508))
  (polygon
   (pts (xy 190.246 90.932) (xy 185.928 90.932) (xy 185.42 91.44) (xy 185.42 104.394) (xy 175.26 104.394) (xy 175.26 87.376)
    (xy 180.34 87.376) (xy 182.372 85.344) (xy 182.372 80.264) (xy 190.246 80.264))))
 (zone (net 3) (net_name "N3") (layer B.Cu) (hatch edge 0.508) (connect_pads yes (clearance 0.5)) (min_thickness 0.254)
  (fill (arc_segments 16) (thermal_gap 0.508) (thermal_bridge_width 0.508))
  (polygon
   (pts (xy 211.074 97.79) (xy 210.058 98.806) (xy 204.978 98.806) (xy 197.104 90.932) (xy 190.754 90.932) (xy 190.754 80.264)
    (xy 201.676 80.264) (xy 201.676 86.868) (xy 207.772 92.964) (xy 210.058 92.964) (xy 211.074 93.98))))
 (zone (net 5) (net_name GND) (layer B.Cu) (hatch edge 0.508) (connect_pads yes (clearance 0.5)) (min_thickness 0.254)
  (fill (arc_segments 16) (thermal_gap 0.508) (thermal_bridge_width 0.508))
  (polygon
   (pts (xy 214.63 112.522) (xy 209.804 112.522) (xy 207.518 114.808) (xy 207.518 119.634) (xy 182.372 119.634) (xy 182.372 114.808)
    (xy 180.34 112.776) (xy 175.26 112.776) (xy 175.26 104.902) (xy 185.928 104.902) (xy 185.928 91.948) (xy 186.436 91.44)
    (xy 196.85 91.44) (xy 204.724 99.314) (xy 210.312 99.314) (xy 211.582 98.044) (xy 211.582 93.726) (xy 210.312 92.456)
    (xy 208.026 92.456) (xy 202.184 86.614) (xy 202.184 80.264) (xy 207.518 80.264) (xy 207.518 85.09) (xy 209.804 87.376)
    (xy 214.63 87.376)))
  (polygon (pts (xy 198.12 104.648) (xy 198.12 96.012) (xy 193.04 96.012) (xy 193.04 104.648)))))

